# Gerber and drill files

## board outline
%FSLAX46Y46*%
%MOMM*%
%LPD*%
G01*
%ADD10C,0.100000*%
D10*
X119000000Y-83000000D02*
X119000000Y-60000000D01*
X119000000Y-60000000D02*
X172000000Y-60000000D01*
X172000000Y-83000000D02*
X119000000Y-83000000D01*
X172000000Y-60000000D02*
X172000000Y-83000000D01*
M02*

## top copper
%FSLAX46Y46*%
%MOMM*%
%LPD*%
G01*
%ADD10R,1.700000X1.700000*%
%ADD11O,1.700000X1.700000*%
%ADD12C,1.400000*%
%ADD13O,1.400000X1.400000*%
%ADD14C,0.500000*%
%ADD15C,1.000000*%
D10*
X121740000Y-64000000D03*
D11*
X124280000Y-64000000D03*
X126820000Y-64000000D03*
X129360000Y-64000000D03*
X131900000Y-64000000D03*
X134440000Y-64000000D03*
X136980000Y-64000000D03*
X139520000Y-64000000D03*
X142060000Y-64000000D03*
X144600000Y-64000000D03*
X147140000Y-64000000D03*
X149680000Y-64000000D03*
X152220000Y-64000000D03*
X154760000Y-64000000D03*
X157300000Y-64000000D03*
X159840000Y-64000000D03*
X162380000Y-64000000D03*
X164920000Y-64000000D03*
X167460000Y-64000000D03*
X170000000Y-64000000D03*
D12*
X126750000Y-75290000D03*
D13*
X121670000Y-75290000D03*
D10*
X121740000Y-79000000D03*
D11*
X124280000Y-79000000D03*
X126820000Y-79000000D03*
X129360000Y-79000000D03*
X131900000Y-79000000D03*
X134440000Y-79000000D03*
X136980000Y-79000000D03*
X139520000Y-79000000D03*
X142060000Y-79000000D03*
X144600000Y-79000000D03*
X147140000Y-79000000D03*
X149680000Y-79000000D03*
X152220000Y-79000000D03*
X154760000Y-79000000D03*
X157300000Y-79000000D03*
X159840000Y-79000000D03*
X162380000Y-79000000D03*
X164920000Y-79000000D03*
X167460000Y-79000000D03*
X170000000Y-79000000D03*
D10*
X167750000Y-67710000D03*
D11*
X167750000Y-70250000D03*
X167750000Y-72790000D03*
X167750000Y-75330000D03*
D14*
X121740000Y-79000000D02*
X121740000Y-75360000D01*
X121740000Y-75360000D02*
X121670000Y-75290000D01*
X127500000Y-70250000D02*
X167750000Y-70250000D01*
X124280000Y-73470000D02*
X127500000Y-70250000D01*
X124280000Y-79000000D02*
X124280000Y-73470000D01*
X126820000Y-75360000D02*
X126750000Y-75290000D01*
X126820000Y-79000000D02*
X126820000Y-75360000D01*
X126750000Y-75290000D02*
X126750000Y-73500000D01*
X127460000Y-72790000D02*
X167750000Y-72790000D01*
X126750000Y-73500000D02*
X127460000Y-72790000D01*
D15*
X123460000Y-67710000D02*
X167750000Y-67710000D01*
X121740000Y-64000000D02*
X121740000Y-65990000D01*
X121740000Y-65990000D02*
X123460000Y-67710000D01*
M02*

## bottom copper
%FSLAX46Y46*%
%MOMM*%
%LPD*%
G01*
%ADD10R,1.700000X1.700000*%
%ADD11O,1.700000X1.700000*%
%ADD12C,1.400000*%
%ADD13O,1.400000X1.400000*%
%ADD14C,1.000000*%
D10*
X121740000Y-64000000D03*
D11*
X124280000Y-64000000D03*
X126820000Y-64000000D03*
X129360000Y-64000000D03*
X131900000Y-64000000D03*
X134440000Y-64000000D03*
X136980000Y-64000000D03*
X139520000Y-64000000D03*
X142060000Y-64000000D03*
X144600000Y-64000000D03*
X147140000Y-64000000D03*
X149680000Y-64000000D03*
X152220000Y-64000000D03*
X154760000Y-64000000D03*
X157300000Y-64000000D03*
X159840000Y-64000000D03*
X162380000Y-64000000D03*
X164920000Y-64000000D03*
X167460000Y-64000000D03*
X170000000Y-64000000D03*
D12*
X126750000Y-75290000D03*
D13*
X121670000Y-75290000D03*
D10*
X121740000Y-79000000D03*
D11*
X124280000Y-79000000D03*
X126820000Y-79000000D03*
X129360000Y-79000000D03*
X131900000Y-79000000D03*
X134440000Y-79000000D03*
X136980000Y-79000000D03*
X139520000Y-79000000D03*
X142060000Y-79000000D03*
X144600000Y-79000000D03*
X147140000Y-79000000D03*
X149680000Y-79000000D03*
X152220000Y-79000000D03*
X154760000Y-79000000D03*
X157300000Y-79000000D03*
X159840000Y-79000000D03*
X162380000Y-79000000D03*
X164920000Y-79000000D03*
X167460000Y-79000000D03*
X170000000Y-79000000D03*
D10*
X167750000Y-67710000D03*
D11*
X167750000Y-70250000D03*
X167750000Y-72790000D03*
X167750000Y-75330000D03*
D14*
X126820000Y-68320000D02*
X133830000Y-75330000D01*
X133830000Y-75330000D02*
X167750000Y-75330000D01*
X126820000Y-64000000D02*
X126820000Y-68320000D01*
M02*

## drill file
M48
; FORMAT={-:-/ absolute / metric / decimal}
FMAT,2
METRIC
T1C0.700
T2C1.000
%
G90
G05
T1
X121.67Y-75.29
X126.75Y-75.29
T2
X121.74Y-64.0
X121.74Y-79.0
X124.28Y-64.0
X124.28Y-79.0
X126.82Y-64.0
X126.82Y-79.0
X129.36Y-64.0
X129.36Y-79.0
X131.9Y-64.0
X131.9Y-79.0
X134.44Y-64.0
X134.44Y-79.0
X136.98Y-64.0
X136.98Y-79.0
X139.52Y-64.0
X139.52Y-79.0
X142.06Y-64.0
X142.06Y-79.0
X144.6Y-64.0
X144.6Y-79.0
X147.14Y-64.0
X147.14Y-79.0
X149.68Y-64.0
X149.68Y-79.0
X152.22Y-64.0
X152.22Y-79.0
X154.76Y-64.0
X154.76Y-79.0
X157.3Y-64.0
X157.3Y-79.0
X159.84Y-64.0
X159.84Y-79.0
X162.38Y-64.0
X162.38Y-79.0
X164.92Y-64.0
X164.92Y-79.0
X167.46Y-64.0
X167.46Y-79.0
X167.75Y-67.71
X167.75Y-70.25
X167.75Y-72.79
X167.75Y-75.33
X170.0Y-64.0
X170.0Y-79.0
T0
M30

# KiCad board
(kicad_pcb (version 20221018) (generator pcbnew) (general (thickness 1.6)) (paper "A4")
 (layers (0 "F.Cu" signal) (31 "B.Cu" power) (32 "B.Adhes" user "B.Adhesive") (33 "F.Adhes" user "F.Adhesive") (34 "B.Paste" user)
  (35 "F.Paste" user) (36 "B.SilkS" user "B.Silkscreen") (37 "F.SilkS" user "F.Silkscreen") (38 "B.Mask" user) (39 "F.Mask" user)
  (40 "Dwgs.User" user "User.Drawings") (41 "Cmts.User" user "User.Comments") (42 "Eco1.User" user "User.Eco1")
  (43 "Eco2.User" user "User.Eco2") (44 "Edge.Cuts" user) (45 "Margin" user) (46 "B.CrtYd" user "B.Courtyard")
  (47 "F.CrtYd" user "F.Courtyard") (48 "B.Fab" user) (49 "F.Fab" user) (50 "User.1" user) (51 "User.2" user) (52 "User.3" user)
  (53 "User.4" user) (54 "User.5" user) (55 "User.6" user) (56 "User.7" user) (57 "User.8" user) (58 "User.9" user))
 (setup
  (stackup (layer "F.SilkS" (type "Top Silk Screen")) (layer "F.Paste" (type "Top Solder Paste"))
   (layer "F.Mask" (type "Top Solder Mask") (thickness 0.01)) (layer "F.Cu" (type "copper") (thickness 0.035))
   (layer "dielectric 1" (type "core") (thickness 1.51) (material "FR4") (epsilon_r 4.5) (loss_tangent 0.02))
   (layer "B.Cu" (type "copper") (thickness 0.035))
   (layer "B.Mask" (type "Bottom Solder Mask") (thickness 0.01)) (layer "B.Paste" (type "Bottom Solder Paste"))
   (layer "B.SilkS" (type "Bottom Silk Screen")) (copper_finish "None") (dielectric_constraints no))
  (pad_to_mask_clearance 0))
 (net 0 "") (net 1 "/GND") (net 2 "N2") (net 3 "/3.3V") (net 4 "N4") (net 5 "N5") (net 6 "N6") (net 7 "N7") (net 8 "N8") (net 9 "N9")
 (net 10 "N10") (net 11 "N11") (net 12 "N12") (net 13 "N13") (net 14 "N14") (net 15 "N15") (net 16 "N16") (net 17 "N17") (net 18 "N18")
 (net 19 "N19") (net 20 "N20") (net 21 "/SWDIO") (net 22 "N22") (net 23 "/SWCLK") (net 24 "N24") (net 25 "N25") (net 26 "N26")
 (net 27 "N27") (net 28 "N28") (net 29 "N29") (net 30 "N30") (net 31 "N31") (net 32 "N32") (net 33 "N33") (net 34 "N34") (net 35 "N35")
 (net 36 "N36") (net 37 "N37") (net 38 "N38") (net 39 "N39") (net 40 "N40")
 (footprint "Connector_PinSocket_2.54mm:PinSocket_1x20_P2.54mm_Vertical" (layer "F.Cu") (at 121.74 64 90)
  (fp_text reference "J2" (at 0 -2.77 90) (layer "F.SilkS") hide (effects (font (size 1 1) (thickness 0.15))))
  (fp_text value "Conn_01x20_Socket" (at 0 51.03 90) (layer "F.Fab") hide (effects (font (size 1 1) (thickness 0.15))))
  (pad "1" thru_hole rect (at 0 0 90) (size 1.7 1.7) (drill 1) (layers "*.Cu" "*.Mask") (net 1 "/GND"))
  (pad "2" thru_hole oval (at 0 2.54 90) (size 1.7 1.7) (drill 1) (layers "*.Cu" "*.Mask") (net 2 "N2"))
  (pad "3" thru_hole oval (at 0 5.08 90) (size 1.7 1.7) (drill 1) (layers "*.Cu" "*.Mask") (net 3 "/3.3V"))
  (pad "4" thru_hole oval (at 0 7.62 90) (size 1.7 1.7) (drill 1) (layers "*.Cu" "*.Mask") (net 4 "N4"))
  (pad "5" thru_hole oval (at 0 10.16 90) (size 1.7 1.7) (drill 1) (layers "*.Cu" "*.Mask") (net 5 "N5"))
  (pad "6" thru_hole oval (at 0 12.7 90) (size 1.7 1.7) (drill 1) (layers "*.Cu" "*.Mask") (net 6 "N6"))
  (pad "7" thru_hole oval (at 0 15.24 90) (size 1.7 1.7) (drill 1) (layers "*.Cu" "*.Mask") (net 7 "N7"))
  (pad "8" thru_hole oval (at 0 17.78 90) (size 1.7 1.7) (drill 1) (layers "*.Cu" "*.Mask") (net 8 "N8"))
  (pad "9" thru_hole oval (at 0 20.32 90) (size 1.7 1.7) (drill 1) (layers "*.Cu" "*.Mask") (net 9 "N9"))
  (pad "10" thru_hole oval (at 0 22.86 90) (size 1.7 1.7) (drill 1) (layers "*.Cu" "*.Mask") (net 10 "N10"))
  (pad "11" thru_hole oval (at 0 25.4 90) (size 1.7 1.7) (drill 1) (layers "*.Cu" "*.Mask") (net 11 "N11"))
  (pad "12" thru_hole oval (at 0 27.94 90) (size 1.7 1.7) (drill 1) (layers "*.Cu" "*.Mask") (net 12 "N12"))
  (pad "13" thru_hole oval (at 0 30.48 90) (size 1.7 1.7) (drill 1) (layers "*.Cu" "*.Mask") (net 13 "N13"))
  (pad "14" thru_hole oval (at 0 33.02 90) (size 1.7 1.7) (drill 1) (layers "*.Cu" "*.Mask") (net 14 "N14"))
  (pad "15" thru_hole oval (at 0 35.56 90) (size 1.7 1.7) (drill 1) (layers "*.Cu" "*.Mask") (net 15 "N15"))
  (pad "16" thru_hole oval (at 0 38.1 90) (size 1.7 1.7) (drill 1) (layers "*.Cu" "*.Mask") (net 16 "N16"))
  (pad "17" thru_hole oval (at 0 40.64 90) (size 1.7 1.7) (drill 1) (layers "*.Cu" "*.Mask") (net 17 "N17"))
  (pad "18" thru_hole oval (at 0 43.18 90) (size 1.7 1.7) (drill 1) (layers "*.Cu" "*.Mask") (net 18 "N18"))
  (pad "19" thru_hole oval (at 0 45.72 90) (size 1.7 1.7) (drill 1) (layers "*.Cu" "*.Mask") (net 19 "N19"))
  (pad "20" thru_hole oval (at 0 48.26 90) (size 1.7 1.7) (drill 1) (layers "*.Cu" "*.Mask") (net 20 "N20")))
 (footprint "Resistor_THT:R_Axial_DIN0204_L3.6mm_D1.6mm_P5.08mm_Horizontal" (layer "F.Cu") (at 126.75 75.29 180)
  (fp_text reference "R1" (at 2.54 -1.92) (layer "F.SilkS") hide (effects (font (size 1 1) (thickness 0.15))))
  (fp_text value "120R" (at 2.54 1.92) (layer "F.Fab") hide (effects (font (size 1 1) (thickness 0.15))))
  (pad "1" thru_hole circle (at 0 0 180) (size 1.4 1.4) (drill 0.7) (layers "*.Cu" "*.Mask") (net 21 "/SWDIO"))
  (pad "2" thru_hole oval (at 5.08 0 180) (size 1.4 1.4) (drill 0.7) (layers "*.Cu" "*.Mask") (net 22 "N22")))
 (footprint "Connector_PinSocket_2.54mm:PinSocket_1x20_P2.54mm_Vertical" (layer "F.Cu") (at 121.74 79 90)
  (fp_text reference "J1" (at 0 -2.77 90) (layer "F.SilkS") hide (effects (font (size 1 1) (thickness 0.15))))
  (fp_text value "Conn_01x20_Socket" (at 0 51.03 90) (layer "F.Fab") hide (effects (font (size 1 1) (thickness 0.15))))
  (pad "1" thru_hole rect (at 0 0 90) (size 1.7 1.7) (drill 1) (layers "*.Cu" "*.Mask") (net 22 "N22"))
  (pad "2" thru_hole oval (at 0 2.54 90) (size 1.7 1.7) (drill 1) (layers "*.Cu" "*.Mask") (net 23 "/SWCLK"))
  (pad "3" thru_hole oval (at 0 5.08 90) (size 1.7 1.7) (drill 1) (layers "*.Cu" "*.Mask") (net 21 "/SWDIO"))
  (pad "4" thru_hole oval (at 0 7.62 90) (size 1.7 1.7) (drill 1) (layers "*.Cu" "*.Mask") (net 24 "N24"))
  (pad "5" thru_hole oval (at 0 10.16 90) (size 1.7 1.7) (drill 1) (layers "*.Cu" "*.Mask") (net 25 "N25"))
  (pad "6" thru_hole oval (at 0 12.7 90) (size 1.7 1.7) (drill 1) (layers "*.Cu" "*.Mask") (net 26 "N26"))
  (pad "7" thru_hole oval (at 0 15.24 90) (size 1.7 1.7) (drill 1) (layers "*.Cu" "*.Mask") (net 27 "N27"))
  (pad "8" thru_hole oval (at 0 17.78 90) (size 1.7 1.7) (drill 1) (layers "*.Cu" "*.Mask") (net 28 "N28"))
  (pad "9" thru_hole oval (at 0 20.32 90) (size 1.7 1.7) (drill 1) (layers "*.Cu" "*.Mask") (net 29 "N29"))
  (pad "10" thru_hole oval (at 0 22.86 90) (size 1.7 1.7) (drill 1) (layers "*.Cu" "*.Mask") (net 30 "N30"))
  (pad "11" thru_hole oval (at 0 25.4 90) (size 1.7 1.7) (drill 1) (layers "*.Cu" "*.Mask") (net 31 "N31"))
  (pad "12" thru_hole oval (at 0 27.94 90) (size 1.7 1.7) (drill 1) (layers "*.Cu" "*.Mask") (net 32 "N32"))
  (pad "13" thru_hole oval (at 0 30.48 90) (size 1.7 1.7) (drill 1) (layers "*.Cu" "*.Mask") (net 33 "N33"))
  (pad "14" thru_hole oval (at 0 33.02 90) (size 1.7 1.7) (drill 1) (layers "*.Cu" "*.Mask") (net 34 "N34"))
  (pad "15" thru_hole oval (at 0 35.56 90) (size 1.7 1.7) (drill 1) (layers "*.Cu" "*.Mask") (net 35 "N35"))
  (pad "16" thru_hole oval (at 0 38.1 90) (size 1.7 1.7) (drill 1) (layers "*.Cu" "*.Mask") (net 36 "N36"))
  (pad "17" thru_hole oval (at 0 40.64 90) (size 1.7 1.7) (drill 1) (layers "*.Cu" "*.Mask") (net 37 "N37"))
  (pad "18" thru_hole oval (at 0 43.18 90) (size 1.7 1.7) (drill 1) (layers "*.Cu" "*.Mask") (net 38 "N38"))
  (pad "19" thru_hole oval (at 0 45.72 90) (size 1.7 1.7) (drill 1) (layers "*.Cu" "*.Mask") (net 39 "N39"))
  (pad "20" thru_hole oval (at 0 48.26 90) (size 1.7 1.7) (drill 1) (layers "*.Cu" "*.Mask") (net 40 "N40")))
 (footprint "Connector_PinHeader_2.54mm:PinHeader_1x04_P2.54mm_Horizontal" (layer "F.Cu") (at 167.75 67.71)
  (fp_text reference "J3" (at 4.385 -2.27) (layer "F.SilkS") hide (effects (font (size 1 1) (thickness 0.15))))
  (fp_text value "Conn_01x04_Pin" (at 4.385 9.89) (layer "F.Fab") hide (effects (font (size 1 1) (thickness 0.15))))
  (pad "1" thru_hole rect (at 0 0) (size 1.7 1.7) (drill 1) (layers "*.Cu" "*.Mask") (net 1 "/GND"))
  (pad "2" thru_hole oval (at 0 2.54) (size 1.7 1.7) (drill 1) (layers "*.Cu" "*.Mask") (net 23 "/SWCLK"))
  (pad "3" thru_hole oval (at 0 5.08) (size 1.7 1.7) (drill 1) (layers "*.Cu" "*.Mask") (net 21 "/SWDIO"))
  (pad "4" thru_hole oval (at 0 7.62) (size 1.7 1.7) (drill 1) (layers "*.Cu" "*.Mask") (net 3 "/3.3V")))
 (gr_line (start 119 83) (end 119 60) (stroke (width 0.1) (type default)) (layer "Edge.Cuts"))
 (gr_line (start 119 60) (end 172 60) (stroke (width 0.1) (type default)) (layer "Edge.Cuts"))
 (gr_line (start 172 83) (end 119 83) (stroke (width 0.1) (type default)) (layer "Edge.Cuts"))
 (gr_line (start 172 60) (end 172 83) (stroke (width 0.1) (type default)) (layer "Edge.Cuts"))
 (segment (start 121.74 79) (end 121.74 75.36) (width 0.5) (layer "F.Cu") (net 22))
 (segment (start 121.74 75.36) (end 121.67 75.29) (width 0.5) (layer "F.Cu") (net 22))
 (segment (start 127.5 70.25) (end 167.75 70.25) (width 0.5) (layer "F.Cu") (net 23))
 (segment (start 124.28 73.47) (end 127.5 70.25) (width 0.5) (layer "F.Cu") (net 23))
 (segment (start 124.28 79) (end 124.28 73.47) (width 0.5) (layer "F.Cu") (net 23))
 (segment (start 126.82 75.36) (end 126.75 75.29) (width 0.5) (layer "F.Cu") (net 21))
 (segment (start 126.82 79) (end 126.82 75.36) (width 0.5) (layer "F.Cu") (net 21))
 (segment (start 126.75 75.29) (end 126.75 73.5) (width 0.5) (layer "F.Cu") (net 21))
 (segment (start 127.46 72.79) (end 167.75 72.79) (width 0.5) (layer "F.Cu") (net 21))
 (segment (start 126.75 73.5) (end 127.46 72.79) (width 0.5) (layer "F.Cu") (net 21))
 (segment (start 123.46 67.71) (end 167.75 67.71) (width 1) (layer "F.Cu") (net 1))
 (segment (start 121.74 64) (end 121.74 65.99) (width 1) (layer "F.Cu") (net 1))
 (segment (start 121.74 65.99) (end 123.46 67.71) (width 1) (layer "F.Cu") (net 1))
 (segment (start 126.82 68.32) (end 133.83 75.33) (width 1) (layer "B.Cu") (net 3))
 (segment (start 133.83 75.33) (end 167.75 75.33) (width 1) (layer "B.Cu") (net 3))
 (segment (start 126.82 64) (end 126.82 68.32) (width 1) (layer "B.Cu") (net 3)))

